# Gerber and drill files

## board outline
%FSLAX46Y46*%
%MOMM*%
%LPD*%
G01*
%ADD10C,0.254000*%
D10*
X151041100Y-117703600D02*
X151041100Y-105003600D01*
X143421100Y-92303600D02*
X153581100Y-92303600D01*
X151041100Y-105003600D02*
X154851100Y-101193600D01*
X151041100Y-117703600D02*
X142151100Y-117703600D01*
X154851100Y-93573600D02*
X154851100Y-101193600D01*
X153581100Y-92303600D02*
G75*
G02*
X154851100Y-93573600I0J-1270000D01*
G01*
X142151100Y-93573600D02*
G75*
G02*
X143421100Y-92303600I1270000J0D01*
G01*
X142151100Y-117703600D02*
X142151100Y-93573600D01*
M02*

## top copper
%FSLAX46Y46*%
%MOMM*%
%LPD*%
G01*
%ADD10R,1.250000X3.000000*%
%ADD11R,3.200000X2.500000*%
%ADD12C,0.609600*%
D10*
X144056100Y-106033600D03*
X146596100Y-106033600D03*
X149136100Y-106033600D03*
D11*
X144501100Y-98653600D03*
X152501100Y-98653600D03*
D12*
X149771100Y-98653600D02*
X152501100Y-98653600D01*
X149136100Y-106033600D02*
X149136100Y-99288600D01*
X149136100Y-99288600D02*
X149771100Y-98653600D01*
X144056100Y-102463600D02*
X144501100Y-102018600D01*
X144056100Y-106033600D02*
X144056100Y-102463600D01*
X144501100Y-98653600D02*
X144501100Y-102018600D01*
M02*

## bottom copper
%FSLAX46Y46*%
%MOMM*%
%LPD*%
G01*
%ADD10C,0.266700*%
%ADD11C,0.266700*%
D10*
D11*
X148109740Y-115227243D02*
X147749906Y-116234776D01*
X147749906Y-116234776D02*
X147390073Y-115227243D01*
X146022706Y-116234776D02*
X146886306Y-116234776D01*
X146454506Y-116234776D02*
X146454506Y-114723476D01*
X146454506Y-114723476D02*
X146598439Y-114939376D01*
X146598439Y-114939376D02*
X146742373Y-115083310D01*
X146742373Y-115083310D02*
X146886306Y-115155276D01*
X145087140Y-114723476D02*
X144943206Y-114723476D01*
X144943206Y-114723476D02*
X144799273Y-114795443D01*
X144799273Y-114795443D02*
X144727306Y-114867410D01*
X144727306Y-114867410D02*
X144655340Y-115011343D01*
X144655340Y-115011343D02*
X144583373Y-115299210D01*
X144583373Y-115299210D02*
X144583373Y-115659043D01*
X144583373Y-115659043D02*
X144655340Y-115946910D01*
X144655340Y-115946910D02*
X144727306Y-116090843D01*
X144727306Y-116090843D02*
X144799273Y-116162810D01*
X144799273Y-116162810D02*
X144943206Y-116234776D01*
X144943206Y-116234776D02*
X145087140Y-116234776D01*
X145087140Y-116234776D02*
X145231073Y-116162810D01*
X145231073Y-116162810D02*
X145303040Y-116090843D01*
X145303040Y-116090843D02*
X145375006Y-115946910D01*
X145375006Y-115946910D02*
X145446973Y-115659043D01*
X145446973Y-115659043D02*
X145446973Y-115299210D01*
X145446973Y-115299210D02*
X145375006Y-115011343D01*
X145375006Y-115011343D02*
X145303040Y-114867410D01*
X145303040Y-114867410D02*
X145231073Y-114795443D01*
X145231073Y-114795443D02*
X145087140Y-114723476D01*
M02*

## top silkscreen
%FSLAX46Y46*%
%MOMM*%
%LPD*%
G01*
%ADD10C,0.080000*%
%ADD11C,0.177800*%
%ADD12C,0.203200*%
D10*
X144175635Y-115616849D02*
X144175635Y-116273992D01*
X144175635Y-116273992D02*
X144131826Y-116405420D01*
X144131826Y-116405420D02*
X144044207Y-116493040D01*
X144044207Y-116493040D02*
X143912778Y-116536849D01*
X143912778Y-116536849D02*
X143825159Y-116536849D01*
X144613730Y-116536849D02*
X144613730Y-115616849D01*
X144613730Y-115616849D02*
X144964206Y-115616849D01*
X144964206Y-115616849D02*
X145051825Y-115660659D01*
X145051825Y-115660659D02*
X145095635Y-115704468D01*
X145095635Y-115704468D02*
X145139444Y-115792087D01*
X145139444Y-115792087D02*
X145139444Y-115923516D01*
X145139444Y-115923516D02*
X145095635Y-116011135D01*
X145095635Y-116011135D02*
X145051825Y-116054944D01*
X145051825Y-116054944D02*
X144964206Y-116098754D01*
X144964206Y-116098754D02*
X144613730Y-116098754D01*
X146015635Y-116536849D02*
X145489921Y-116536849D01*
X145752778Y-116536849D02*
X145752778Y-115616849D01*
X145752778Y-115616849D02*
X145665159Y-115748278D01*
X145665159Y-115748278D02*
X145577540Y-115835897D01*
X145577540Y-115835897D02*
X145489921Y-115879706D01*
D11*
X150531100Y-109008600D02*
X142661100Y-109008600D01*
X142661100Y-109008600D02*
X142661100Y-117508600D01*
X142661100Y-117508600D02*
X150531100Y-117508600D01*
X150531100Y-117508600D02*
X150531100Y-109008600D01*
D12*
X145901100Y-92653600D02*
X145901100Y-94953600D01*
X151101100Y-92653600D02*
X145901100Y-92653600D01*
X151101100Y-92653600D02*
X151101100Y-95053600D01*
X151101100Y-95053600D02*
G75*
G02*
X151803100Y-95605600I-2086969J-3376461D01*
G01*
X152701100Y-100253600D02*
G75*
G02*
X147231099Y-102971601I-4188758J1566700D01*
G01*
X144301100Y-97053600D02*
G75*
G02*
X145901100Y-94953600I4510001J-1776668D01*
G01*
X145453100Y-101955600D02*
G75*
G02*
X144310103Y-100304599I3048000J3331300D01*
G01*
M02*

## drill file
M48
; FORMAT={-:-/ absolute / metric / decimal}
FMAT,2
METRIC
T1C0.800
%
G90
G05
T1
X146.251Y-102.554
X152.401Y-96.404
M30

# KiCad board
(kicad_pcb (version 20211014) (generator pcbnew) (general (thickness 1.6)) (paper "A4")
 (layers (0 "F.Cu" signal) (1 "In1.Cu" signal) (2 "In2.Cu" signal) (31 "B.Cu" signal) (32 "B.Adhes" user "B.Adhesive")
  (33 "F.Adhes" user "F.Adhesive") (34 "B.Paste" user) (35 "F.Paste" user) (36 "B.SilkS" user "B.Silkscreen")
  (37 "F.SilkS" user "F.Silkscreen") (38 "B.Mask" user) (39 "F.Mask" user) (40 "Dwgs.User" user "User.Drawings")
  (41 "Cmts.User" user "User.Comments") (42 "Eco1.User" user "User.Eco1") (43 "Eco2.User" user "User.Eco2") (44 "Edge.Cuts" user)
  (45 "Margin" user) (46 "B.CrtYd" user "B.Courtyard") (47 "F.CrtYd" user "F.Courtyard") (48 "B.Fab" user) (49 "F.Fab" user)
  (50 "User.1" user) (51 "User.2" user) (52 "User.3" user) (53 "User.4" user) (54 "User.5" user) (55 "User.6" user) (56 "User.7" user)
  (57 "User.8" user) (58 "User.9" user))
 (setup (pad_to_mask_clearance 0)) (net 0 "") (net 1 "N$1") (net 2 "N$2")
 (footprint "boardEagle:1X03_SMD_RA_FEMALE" (layer "F.Cu") (at 146.5961 113.2586)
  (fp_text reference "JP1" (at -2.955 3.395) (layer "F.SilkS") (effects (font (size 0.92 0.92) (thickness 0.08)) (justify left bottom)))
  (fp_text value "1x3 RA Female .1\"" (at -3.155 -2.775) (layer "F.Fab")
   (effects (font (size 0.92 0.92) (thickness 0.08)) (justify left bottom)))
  (fp_line (start 3.935 -4.25) (end -3.935 -4.25) (layer "F.SilkS") (width 0.1778))
  (fp_line (start -3.935 -4.25) (end -3.935 4.25) (layer "F.SilkS") (width 0.1778))
  (fp_line (start -3.935 4.25) (end 3.935 4.25) (layer "F.SilkS") (width 0.1778))
  (fp_line (start 3.935 4.25) (end 3.935 -4.25) (layer "F.SilkS") (width 0.1778))
  (pad "1" smd rect (at -2.54 -7.225 180) (size 1.25 3) (layers "F.Cu" "F.Paste" "F.Mask") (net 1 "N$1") (solder_mask_margin 0.1016))
  (pad "2" smd rect (at 0 -7.225 180) (size 1.25 3) (layers "F.Cu" "F.Paste" "F.Mask") (solder_mask_margin 0.1016))
  (pad "3" smd rect (at 2.54 -7.225 180) (size 1.25 3) (layers "F.Cu" "F.Paste" "F.Mask") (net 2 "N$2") (solder_mask_margin 0.1016)))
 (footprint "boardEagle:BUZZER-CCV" (layer "F.Cu") (at 148.5011 98.6536 180)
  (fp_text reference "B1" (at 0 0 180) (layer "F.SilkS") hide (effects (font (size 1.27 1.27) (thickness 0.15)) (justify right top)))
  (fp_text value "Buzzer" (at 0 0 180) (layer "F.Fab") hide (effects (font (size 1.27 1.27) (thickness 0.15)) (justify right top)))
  (fp_line (start 2.6 6) (end 2.6 3.7) (layer "F.SilkS") (width 0.2032))
  (fp_line (start -2.6 6) (end 2.6 6) (layer "F.SilkS") (width 0.2032))
  (fp_line (start -2.6 6) (end -2.6 3.6) (layer "F.SilkS") (width 0.2032))
  (fp_arc (start -2.6 3.6) (mid -2.966573 3.343805) (end -3.302 3.048) (layer "F.SilkS") (width 0.2032))
  (fp_arc (start -4.2 -1.6) (mid -2.00129 -4.038291) (end 1.270001 -4.318001) (layer "F.SilkS") (width 0.2032))
  (fp_arc (start 4.2 1.6) (mid 3.545723 2.761027) (end 2.6 3.7) (layer "F.SilkS") (width 0.2032))
  (fp_arc (start 3.048 -3.302) (mid 3.712443 -2.540845) (end 4.191 -1.651) (layer "F.SilkS") (width 0.2032))
  (pad "" np_thru_hole circle (at 2.25 -3.9 180) (size 0.8 0.8) (drill 0.8) (layers *.Cu *.Mask))
  (pad "" np_thru_hole circle (at -3.9 2.25 180) (size 0.8 0.8) (drill 0.8) (layers *.Cu *.Mask))
  (pad "+" smd rect (at 4 0 180) (size 3.2 2.5) (layers "F.Cu" "F.Paste" "F.Mask") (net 1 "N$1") (solder_mask_margin 0.1016))
  (pad "-" smd rect (at -4 0 180) (size 3.2 2.5) (layers "F.Cu" "F.Paste" "F.Mask") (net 2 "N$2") (solder_mask_margin 0.1016)))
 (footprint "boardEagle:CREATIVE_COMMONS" (layer "F.Cu") (at 144.6911 132.9436)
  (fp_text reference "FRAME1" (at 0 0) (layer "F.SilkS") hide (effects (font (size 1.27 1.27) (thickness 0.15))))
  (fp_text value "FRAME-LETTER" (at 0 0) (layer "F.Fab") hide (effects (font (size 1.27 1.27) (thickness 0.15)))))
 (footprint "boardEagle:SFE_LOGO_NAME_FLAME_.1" (layer "B.Cu") (at 153.9621 103.2256 180)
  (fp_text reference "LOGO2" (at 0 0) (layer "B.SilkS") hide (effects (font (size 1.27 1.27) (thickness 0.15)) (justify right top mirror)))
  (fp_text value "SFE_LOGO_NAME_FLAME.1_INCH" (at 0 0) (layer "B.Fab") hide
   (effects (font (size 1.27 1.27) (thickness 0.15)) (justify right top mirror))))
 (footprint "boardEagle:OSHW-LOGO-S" (layer "B.Cu") (at 144.3101 105.0036 180)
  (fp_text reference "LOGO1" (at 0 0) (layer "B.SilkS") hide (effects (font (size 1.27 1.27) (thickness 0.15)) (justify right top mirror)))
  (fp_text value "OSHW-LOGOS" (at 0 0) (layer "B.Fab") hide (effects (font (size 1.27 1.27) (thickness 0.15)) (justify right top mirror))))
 (gr_line (start 151.0411 117.7036) (end 151.0411 105.0036) (layer "Edge.Cuts") (width 0.254))
 (gr_line (start 143.4211 92.3036) (end 153.5811 92.3036) (layer "Edge.Cuts") (width 0.254))
 (gr_line (start 151.0411 105.0036) (end 154.8511 101.1936) (layer "Edge.Cuts") (width 0.254))
 (gr_line (start 151.0411 117.7036) (end 142.1511 117.7036) (layer "Edge.Cuts") (width 0.254))
 (gr_line (start 154.8511 93.5736) (end 154.8511 101.1936) (layer "Edge.Cuts") (width 0.254))
 (gr_arc (start 153.5811 92.3036) (mid 154.479126 92.675574) (end 154.8511 93.5736) (layer "Edge.Cuts") (width 0.254))
 (gr_arc (start 142.1511 93.5736) (mid 142.523074 92.675574) (end 143.4211 92.3036) (layer "Edge.Cuts") (width 0.254))
 (gr_line (start 142.1511 117.7036) (end 142.1511 93.5736) (layer "Edge.Cuts") (width 0.254))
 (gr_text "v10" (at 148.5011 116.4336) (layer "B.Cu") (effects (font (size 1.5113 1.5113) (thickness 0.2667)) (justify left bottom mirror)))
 (segment (start 149.7711 98.6536) (end 152.5011 98.6536) (width 0.6096) (layer "F.Cu") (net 2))
 (segment (start 149.1361 106.0336) (end 149.1361 99.2886) (width 0.6096) (layer "F.Cu") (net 2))
 (segment (start 149.1361 99.2886) (end 149.7711 98.6536) (width 0.6096) (layer "F.Cu") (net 2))
 (segment (start 144.0561 102.4636) (end 144.5011 102.0186) (width 0.6096) (layer "F.Cu") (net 1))
 (segment (start 144.0561 106.0336) (end 144.0561 102.4636) (width 0.6096) (layer "F.Cu") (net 1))
 (segment (start 144.5011 98.6536) (end 144.5011 102.0186) (width 0.6096) (layer "F.Cu") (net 1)))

